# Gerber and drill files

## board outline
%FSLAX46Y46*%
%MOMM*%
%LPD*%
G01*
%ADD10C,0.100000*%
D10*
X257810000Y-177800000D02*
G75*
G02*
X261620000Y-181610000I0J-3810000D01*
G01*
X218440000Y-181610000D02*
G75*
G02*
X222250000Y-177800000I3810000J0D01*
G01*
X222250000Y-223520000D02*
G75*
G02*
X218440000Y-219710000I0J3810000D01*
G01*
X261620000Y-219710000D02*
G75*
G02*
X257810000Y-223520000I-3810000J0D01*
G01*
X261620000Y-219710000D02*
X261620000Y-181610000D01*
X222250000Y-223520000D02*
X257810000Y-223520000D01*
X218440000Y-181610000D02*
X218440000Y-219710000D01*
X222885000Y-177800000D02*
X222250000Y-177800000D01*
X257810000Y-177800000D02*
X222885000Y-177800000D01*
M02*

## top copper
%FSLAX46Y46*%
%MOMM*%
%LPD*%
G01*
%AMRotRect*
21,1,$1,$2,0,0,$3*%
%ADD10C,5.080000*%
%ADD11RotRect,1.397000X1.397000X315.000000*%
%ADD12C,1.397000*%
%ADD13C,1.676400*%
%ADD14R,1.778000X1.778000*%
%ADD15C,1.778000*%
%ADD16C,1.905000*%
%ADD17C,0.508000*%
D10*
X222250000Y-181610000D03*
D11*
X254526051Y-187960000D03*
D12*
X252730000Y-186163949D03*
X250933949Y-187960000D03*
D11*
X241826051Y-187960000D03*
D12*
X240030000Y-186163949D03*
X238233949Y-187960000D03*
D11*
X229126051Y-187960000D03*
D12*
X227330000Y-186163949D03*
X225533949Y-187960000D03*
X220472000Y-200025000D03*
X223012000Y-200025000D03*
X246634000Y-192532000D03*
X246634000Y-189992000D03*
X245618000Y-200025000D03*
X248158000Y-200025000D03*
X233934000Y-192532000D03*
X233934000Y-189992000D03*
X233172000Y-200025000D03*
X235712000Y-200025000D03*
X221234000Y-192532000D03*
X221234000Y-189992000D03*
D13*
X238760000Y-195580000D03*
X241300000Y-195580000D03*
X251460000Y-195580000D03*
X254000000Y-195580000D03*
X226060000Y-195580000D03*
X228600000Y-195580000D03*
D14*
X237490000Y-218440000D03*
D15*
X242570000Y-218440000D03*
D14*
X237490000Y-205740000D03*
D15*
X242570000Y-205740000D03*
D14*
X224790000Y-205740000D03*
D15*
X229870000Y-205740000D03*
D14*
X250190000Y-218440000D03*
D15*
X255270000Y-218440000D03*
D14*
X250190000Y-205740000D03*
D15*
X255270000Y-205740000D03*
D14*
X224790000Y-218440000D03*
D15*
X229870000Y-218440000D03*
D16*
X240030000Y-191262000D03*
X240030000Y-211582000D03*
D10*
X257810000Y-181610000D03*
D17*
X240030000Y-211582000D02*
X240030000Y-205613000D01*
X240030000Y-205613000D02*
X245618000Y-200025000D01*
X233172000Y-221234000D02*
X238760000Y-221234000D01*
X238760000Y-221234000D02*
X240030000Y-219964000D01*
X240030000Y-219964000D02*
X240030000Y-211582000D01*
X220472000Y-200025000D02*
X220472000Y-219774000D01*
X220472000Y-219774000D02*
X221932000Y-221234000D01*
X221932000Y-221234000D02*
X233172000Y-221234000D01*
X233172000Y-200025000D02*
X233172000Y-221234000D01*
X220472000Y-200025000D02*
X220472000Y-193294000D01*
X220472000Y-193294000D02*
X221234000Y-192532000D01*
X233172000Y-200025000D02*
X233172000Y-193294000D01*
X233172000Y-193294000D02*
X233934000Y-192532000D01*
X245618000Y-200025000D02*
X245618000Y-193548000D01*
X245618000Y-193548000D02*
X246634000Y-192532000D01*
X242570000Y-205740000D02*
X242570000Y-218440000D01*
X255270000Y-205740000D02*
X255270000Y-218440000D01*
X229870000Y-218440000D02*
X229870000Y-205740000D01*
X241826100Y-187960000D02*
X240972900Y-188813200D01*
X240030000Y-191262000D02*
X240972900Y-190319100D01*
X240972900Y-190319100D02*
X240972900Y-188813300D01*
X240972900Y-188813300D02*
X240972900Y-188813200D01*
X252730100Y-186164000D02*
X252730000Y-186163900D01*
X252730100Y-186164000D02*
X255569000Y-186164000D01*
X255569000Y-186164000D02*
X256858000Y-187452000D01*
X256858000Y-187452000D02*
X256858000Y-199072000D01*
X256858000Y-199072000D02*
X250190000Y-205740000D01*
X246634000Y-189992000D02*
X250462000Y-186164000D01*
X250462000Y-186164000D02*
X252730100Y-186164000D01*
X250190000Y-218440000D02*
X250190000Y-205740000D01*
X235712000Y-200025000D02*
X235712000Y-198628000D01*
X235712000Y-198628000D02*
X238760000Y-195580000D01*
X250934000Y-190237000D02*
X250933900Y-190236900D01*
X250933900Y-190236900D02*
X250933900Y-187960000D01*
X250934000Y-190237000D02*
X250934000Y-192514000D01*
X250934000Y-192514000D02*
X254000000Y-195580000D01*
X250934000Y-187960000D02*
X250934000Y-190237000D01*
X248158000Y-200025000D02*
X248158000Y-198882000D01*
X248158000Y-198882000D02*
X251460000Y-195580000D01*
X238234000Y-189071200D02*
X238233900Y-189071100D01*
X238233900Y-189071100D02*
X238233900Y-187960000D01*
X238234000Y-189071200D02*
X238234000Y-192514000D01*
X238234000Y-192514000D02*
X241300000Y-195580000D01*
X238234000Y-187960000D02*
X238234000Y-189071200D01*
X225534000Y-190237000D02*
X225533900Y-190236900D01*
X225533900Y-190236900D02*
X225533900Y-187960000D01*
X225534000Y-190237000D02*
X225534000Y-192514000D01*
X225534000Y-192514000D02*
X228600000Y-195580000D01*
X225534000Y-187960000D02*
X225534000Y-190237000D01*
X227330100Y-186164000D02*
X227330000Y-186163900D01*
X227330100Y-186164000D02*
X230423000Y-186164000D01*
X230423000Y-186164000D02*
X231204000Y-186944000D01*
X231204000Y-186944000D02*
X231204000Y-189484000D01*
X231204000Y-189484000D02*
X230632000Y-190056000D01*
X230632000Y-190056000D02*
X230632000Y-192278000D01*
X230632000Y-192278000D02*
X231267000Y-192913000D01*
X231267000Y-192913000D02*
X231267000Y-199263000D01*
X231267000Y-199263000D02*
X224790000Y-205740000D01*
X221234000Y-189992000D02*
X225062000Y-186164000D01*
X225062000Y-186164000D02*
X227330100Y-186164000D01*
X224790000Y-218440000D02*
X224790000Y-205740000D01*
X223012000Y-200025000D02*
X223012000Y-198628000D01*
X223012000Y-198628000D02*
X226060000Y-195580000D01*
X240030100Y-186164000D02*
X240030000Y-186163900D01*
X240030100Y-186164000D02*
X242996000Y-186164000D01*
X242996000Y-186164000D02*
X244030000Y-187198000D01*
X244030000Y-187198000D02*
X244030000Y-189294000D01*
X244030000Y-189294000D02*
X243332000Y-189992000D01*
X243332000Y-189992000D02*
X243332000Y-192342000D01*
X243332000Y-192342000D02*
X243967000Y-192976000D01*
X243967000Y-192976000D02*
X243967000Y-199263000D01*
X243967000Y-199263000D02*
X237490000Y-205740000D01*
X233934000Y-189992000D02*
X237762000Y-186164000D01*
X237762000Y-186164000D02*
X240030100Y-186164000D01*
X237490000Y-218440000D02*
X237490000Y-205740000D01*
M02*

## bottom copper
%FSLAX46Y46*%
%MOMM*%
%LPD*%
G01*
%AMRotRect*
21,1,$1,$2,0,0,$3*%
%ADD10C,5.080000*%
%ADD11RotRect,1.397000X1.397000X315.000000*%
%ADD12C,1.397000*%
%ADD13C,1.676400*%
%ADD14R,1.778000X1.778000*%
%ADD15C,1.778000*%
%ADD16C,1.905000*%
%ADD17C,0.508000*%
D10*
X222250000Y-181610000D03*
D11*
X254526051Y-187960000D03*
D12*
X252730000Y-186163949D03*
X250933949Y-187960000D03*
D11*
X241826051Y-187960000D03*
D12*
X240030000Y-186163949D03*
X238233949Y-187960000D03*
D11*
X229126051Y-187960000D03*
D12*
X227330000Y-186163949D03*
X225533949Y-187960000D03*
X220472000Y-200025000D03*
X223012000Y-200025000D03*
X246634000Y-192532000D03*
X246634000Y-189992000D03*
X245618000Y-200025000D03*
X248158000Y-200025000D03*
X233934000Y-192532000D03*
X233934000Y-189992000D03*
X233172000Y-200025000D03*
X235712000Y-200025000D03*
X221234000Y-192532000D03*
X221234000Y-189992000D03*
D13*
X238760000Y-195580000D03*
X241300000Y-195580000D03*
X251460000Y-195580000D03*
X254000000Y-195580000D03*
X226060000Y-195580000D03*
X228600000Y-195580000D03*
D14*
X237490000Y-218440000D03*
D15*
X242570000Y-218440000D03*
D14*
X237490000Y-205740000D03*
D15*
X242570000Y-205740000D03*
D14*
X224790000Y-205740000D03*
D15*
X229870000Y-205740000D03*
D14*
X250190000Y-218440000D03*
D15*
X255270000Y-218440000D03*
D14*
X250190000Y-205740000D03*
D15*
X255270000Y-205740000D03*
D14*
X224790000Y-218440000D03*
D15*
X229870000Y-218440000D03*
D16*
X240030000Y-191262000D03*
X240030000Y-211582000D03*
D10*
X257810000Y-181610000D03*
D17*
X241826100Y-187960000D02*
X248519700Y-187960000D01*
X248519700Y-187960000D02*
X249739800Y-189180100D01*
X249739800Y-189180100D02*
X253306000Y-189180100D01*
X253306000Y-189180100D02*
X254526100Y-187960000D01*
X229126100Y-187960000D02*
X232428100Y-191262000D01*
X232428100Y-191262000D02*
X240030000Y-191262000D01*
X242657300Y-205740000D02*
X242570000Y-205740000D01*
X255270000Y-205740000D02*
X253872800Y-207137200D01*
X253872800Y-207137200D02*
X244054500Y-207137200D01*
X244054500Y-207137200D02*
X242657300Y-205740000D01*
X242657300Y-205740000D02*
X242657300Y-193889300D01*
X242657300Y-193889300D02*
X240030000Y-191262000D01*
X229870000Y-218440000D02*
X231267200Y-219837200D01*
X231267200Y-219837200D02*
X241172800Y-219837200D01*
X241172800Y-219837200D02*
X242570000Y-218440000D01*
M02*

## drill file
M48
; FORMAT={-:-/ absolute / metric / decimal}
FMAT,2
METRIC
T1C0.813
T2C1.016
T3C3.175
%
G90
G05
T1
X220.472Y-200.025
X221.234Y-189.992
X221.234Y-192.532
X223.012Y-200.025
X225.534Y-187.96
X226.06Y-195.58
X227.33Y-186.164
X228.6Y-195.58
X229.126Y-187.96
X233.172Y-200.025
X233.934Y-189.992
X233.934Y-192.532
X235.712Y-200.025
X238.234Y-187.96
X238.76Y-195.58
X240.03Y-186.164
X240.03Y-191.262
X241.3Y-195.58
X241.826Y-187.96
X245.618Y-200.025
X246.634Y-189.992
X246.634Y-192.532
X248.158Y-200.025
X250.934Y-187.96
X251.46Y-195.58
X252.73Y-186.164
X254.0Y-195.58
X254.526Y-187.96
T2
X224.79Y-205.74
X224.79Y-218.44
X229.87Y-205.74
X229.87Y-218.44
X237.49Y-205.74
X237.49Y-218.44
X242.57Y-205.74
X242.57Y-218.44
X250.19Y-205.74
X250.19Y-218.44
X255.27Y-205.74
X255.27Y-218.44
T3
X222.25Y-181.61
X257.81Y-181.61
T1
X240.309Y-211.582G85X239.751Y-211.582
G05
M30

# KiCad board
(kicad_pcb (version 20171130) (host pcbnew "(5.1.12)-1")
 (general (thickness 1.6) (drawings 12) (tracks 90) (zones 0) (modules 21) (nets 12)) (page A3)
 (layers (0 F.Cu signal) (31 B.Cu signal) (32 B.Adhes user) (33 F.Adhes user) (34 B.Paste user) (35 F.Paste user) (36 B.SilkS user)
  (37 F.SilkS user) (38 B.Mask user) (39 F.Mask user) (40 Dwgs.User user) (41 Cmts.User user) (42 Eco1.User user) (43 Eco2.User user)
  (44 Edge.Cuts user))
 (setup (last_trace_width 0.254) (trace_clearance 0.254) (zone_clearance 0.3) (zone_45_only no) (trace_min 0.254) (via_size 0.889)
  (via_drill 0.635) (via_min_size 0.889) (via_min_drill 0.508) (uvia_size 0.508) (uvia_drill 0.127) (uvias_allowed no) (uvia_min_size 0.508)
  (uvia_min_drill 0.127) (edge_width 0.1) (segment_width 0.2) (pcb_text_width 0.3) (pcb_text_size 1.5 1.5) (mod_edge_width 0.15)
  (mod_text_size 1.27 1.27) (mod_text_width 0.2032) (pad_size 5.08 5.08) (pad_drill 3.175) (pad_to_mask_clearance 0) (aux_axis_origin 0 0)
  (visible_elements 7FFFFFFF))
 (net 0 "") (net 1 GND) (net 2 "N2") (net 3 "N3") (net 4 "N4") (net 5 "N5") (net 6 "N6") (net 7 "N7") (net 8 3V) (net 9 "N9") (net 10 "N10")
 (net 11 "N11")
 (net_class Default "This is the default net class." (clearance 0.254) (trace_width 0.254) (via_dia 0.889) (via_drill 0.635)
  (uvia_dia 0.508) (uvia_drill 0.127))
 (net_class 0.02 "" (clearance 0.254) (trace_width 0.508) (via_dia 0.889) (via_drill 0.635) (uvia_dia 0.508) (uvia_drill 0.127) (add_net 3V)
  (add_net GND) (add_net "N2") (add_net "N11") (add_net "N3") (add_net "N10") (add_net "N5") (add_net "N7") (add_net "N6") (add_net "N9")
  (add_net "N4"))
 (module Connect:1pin (layer F.Cu) (at 222.25 181.61)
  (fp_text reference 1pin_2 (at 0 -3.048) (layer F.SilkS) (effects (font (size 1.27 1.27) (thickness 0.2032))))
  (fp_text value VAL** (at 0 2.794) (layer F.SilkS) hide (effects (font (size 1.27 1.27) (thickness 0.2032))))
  (pad 1 thru_hole circle (at 0 0) (size 5.08 5.08) (drill 3.175) (layers *.Cu *.Mask F.SilkS)))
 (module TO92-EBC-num (layer F.Cu) (at 252.73 187.96 315)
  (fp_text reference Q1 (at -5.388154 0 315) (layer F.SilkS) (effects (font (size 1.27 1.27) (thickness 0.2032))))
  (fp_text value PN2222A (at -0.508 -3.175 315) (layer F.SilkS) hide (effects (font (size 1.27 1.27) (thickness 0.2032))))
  (pad 1 thru_hole rect (at 1.27 -1.27 315) (size 1.397 1.397) (drill 0.8128) (layers *.Cu *.Mask F.SilkS) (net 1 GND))
  (pad 2 thru_hole circle (at -1.27 -1.27 315) (size 1.397 1.397) (drill 0.8128) (layers *.Cu *.Mask F.SilkS) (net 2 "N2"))
  (pad 3 thru_hole circle (at -1.27 1.27 315) (size 1.397 1.397) (drill 0.8128) (layers *.Cu *.Mask F.SilkS) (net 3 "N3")))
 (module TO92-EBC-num (layer F.Cu) (at 240.03 187.96 315)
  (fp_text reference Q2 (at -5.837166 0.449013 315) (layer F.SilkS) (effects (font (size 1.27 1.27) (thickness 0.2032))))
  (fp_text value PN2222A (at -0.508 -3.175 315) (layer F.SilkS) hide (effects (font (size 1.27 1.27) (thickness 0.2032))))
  (pad 1 thru_hole rect (at 1.27 -1.27 315) (size 1.397 1.397) (drill 0.8128) (layers *.Cu *.Mask F.SilkS) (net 1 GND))
  (pad 2 thru_hole circle (at -1.27 -1.27 315) (size 1.397 1.397) (drill 0.8128) (layers *.Cu *.Mask F.SilkS) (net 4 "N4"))
  (pad 3 thru_hole circle (at -1.27 1.27 315) (size 1.397 1.397) (drill 0.8128) (layers *.Cu *.Mask F.SilkS) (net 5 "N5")))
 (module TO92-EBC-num (layer F.Cu) (at 227.33 187.96 315)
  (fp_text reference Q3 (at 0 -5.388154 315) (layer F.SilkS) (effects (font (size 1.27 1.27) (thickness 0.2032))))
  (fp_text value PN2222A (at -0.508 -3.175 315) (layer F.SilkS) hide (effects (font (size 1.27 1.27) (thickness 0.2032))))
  (pad 1 thru_hole rect (at 1.27 -1.27 315) (size 1.397 1.397) (drill 0.8128) (layers *.Cu *.Mask F.SilkS) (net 1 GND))
  (pad 2 thru_hole circle (at -1.27 -1.27 315) (size 1.397 1.397) (drill 0.8128) (layers *.Cu *.Mask F.SilkS) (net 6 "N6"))
  (pad 3 thru_hole circle (at -1.27 1.27 315) (size 1.397 1.397) (drill 0.8128) (layers *.Cu *.Mask F.SilkS) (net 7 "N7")))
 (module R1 (layer F.Cu) (at 221.742 200.025) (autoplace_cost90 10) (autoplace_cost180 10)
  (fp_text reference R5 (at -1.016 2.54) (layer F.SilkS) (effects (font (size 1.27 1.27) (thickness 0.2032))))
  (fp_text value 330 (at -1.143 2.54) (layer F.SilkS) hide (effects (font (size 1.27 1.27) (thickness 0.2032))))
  (pad 1 thru_hole circle (at -1.27 0) (size 1.397 1.397) (drill 0.8128) (layers *.Cu *.Mask F.SilkS) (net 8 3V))
  (pad 2 thru_hole circle (at 1.27 0) (size 1.397 1.397) (drill 0.8128) (layers *.Cu *.Mask F.SilkS) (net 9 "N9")))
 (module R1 (layer F.Cu) (at 246.634 191.262 90) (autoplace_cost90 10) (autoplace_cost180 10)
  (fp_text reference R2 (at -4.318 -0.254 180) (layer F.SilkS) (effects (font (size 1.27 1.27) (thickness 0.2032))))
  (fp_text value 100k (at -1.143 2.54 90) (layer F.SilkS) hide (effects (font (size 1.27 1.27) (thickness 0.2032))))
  (pad 1 thru_hole circle (at -1.27 0 90) (size 1.397 1.397) (drill 0.8128) (layers *.Cu *.Mask F.SilkS) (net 8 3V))
  (pad 2 thru_hole circle (at 1.27 0 90) (size 1.397 1.397) (drill 0.8128) (layers *.Cu *.Mask F.SilkS) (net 2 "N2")))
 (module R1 (layer F.Cu) (at 246.888 200.025) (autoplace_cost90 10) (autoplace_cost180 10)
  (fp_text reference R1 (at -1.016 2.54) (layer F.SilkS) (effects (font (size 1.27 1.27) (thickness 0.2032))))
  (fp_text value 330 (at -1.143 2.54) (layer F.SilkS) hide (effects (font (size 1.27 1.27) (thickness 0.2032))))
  (pad 1 thru_hole circle (at -1.27 0) (size 1.397 1.397) (drill 0.8128) (layers *.Cu *.Mask F.SilkS) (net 8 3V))
  (pad 2 thru_hole circle (at 1.27 0) (size 1.397 1.397) (drill 0.8128) (layers *.Cu *.Mask F.SilkS) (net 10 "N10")))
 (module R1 (layer F.Cu) (at 233.934 191.262 90) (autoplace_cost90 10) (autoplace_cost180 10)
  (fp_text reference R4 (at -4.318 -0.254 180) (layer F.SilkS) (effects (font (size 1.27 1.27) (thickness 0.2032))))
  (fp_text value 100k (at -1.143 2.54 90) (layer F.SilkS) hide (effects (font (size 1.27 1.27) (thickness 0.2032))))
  (pad 1 thru_hole circle (at -1.27 0 90) (size 1.397 1.397) (drill 0.8128) (layers *.Cu *.Mask F.SilkS) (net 8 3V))
  (pad 2 thru_hole circle (at 1.27 0 90) (size 1.397 1.397) (drill 0.8128) (layers *.Cu *.Mask F.SilkS) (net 4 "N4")))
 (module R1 (layer F.Cu) (at 234.442 200.025) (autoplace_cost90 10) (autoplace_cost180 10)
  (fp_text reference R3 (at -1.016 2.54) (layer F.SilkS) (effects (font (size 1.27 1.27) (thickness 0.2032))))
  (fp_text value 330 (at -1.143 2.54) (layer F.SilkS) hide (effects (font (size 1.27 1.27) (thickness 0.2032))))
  (pad 1 thru_hole circle (at -1.27 0) (size 1.397 1.397) (drill 0.8128) (layers *.Cu *.Mask F.SilkS) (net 8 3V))
  (pad 2 thru_hole circle (at 1.27 0) (size 1.397 1.397) (drill 0.8128) (layers *.Cu *.Mask F.SilkS) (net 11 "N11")))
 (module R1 (layer F.Cu) (at 221.234 191.262 90) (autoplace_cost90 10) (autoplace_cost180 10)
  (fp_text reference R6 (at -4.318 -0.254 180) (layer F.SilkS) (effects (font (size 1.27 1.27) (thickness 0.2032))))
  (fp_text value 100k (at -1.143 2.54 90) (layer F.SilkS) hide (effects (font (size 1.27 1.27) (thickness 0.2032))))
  (pad 1 thru_hole circle (at -1.27 0 90) (size 1.397 1.397) (drill 0.8128) (layers *.Cu *.Mask F.SilkS) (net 8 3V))
  (pad 2 thru_hole circle (at 1.27 0 90) (size 1.397 1.397) (drill 0.8128) (layers *.Cu *.Mask F.SilkS) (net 6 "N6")))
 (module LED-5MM (layer F.Cu) (at 240.03 195.58)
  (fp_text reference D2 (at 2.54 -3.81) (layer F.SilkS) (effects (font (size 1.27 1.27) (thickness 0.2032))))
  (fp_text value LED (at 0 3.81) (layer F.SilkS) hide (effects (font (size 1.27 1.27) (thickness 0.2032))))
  (pad 1 thru_hole circle (at -1.27 0) (size 1.6764 1.6764) (drill 0.8128) (layers *.Cu *.Mask F.SilkS) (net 11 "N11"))
  (pad 2 thru_hole circle (at 1.27 0) (size 1.6764 1.6764) (drill 0.8128) (layers *.Cu *.Mask F.SilkS) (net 5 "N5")))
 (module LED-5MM (layer F.Cu) (at 252.73 195.58)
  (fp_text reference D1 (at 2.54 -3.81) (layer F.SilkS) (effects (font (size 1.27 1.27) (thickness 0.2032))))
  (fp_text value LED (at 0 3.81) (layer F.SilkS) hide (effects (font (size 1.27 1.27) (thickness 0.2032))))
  (pad 1 thru_hole circle (at -1.27 0) (size 1.6764 1.6764) (drill 0.8128) (layers *.Cu *.Mask F.SilkS) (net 10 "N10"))
  (pad 2 thru_hole circle (at 1.27 0) (size 1.6764 1.6764) (drill 0.8128) (layers *.Cu *.Mask F.SilkS) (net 3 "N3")))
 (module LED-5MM (layer F.Cu) (at 227.33 195.58)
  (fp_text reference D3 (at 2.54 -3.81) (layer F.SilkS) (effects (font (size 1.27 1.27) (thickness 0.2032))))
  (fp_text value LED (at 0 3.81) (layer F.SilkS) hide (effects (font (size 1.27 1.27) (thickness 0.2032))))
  (pad 1 thru_hole circle (at -1.27 0) (size 1.6764 1.6764) (drill 0.8128) (layers *.Cu *.Mask F.SilkS) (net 9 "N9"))
  (pad 2 thru_hole circle (at 1.27 0) (size 1.6764 1.6764) (drill 0.8128) (layers *.Cu *.Mask F.SilkS) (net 7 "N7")))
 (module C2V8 (layer F.Cu) (at 240.03 218.44)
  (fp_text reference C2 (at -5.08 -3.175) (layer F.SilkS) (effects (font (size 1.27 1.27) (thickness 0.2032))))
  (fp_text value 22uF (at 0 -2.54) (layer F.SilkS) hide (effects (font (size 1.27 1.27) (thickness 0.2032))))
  (pad 1 thru_hole rect (at -2.54 0) (size 1.778 1.778) (drill 1.016) (layers *.Cu *.Mask F.SilkS) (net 4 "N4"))
  (pad 2 thru_hole circle (at 2.54 0) (size 1.778 1.778) (drill 1.016) (layers *.Cu *.Mask F.SilkS) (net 1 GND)))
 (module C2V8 (layer F.Cu) (at 240.03 205.74)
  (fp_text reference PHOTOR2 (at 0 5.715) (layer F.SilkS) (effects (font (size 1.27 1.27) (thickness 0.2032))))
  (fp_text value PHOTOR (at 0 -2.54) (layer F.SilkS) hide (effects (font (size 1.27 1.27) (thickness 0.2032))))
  (pad 1 thru_hole rect (at -2.54 0) (size 1.778 1.778) (drill 1.016) (layers *.Cu *.Mask F.SilkS) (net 4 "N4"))
  (pad 2 thru_hole circle (at 2.54 0) (size 1.778 1.778) (drill 1.016) (layers *.Cu *.Mask F.SilkS) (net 1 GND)))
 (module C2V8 (layer F.Cu) (at 227.33 205.74)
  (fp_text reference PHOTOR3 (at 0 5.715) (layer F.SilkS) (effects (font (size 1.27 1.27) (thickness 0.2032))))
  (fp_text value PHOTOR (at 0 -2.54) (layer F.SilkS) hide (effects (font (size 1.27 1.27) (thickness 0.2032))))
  (pad 1 thru_hole rect (at -2.54 0) (size 1.778 1.778) (drill 1.016) (layers *.Cu *.Mask F.SilkS) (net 6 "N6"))
  (pad 2 thru_hole circle (at 2.54 0) (size 1.778 1.778) (drill 1.016) (layers *.Cu *.Mask F.SilkS) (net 1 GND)))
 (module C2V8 (layer F.Cu) (at 252.73 218.44)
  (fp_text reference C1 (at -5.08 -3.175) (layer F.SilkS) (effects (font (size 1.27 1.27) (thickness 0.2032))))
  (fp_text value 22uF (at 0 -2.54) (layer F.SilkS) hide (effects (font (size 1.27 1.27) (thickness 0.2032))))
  (pad 1 thru_hole rect (at -2.54 0) (size 1.778 1.778) (drill 1.016) (layers *.Cu *.Mask F.SilkS) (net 2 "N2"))
  (pad 2 thru_hole circle (at 2.54 0) (size 1.778 1.778) (drill 1.016) (layers *.Cu *.Mask F.SilkS) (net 1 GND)))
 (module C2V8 (layer F.Cu) (at 252.73 205.74)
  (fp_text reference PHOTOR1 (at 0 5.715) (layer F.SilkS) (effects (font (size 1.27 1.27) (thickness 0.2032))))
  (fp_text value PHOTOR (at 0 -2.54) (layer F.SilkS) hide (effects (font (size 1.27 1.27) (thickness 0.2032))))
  (pad 1 thru_hole rect (at -2.54 0) (size 1.778 1.778) (drill 1.016) (layers *.Cu *.Mask F.SilkS) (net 2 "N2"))
  (pad 2 thru_hole circle (at 2.54 0) (size 1.778 1.778) (drill 1.016) (layers *.Cu *.Mask F.SilkS) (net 1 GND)))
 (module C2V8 (layer F.Cu) (at 227.33 218.44)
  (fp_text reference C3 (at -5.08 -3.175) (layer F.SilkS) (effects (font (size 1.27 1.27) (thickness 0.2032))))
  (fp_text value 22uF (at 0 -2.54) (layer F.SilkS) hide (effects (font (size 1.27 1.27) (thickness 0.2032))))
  (pad 1 thru_hole rect (at -2.54 0) (size 1.778 1.778) (drill 1.016) (layers *.Cu *.Mask F.SilkS) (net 6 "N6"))
  (pad 2 thru_hole circle (at 2.54 0) (size 1.778 1.778) (drill 1.016) (layers *.Cu *.Mask F.SilkS) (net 1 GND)))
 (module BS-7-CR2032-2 (layer B.Cu) (at 240.03 195.072 270)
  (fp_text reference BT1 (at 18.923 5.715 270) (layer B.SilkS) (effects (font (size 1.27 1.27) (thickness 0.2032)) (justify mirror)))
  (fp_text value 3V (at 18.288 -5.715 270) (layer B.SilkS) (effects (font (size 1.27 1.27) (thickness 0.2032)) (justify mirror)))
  (pad 2 thru_hole circle (at -3.81 0 270) (size 1.905 1.905) (drill 0.8128) (layers *.Cu *.Mask B.SilkS) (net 1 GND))
  (pad 1 thru_hole circle (at 16.51 0 270) (size 1.905 1.905) (drill oval 0.8128 1.3716) (layers *.Cu *.Mask B.SilkS) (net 8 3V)))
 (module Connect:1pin (layer F.Cu) (at 257.81 181.61)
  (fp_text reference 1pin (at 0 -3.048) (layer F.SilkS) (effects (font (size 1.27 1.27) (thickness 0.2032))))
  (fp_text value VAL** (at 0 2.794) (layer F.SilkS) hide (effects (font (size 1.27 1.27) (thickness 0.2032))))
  (pad 1 thru_hole circle (at 0 0) (size 5.08 5.08) (drill 3.175) (layers *.Cu *.Mask F.SilkS)))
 (gr_arc (start 257.81 181.61) (end 257.81 177.8) (angle 90) (layer Edge.Cuts) (width 0.1))
 (gr_arc (start 222.25 181.61) (end 218.44 181.61) (angle 90) (layer Edge.Cuts) (width 0.1))
 (gr_arc (start 222.25 219.71) (end 222.25 223.52) (angle 90) (layer Edge.Cuts) (width 0.1))
 (gr_arc (start 257.81 219.71) (end 261.62 219.71) (angle 90) (layer Edge.Cuts) (width 0.1))
 (gr_line (start 261.62 219.71) (end 261.62 181.61) (angle 90) (layer Edge.Cuts) (width 0.1))
 (gr_line (start 222.25 223.52) (end 257.81 223.52) (angle 90) (layer Edge.Cuts) (width 0.1))
 (gr_line (start 218.44 181.61) (end 218.44 219.71) (angle 90) (layer Edge.Cuts) (width 0.1))
 (gr_line (start 222.885 177.8) (end 222.25 177.8) (angle 90) (layer Edge.Cuts) (width 0.1))
 (gr_line (start 257.81 177.8) (end 222.885 177.8) (angle 90) (layer Edge.Cuts) (width 0.1))
 (segment (start 240.03 211.582) (end 240.03 205.613) (width 0.508) (layer F.Cu) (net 8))
 (segment (start 240.03 205.613) (end 245.618 200.025) (width 0.508) (layer F.Cu) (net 8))
 (segment (start 233.172 221.234) (end 238.76 221.234) (width 0.508) (layer F.Cu) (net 8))
 (segment (start 238.76 221.234) (end 240.03 219.964) (width 0.508) (layer F.Cu) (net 8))
 (segment (start 240.03 219.964) (end 240.03 211.582) (width 0.508) (layer F.Cu) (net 8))
 (segment (start 220.472 200.025) (end 220.472 219.774) (width 0.508) (layer F.Cu) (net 8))
 (segment (start 220.472 219.774) (end 221.932 221.234) (width 0.508) (layer F.Cu) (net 8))
 (segment (start 221.932 221.234) (end 233.172 221.234) (width 0.508) (layer F.Cu) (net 8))
 (segment (start 233.172 200.025) (end 233.172 221.234) (width 0.508) (layer F.Cu) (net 8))
 (segment (start 220.472 200.025) (end 220.472 193.294) (width 0.508) (layer F.Cu) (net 8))
 (segment (start 220.472 193.294) (end 221.234 192.532) (width 0.508) (layer F.Cu) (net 8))
 (segment (start 233.172 200.025) (end 233.172 193.294) (width 0.508) (layer F.Cu) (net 8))
 (segment (start 233.172 193.294) (end 233.934 192.532) (width 0.508) (layer F.Cu) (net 8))
 (segment (start 245.618 200.025) (end 245.618 193.548) (width 0.508) (layer F.Cu) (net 8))
 (segment (start 245.618 193.548) (end 246.634 192.532) (width 0.508) (layer F.Cu) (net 8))
 (segment (start 241.8261 187.96) (end 248.5197 187.96) (width 0.508) (layer B.Cu) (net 1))
 (segment (start 248.5197 187.96) (end 249.7398 189.1801) (width 0.508) (layer B.Cu) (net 1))
 (segment (start 249.7398 189.1801) (end 253.306 189.1801) (width 0.508) (layer B.Cu) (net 1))
 (segment (start 253.306 189.1801) (end 254.5261 187.96) (width 0.508) (layer B.Cu) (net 1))
 (segment (start 229.1261 187.96) (end 232.4281 191.262) (width 0.508) (layer B.Cu) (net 1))
 (segment (start 232.4281 191.262) (end 240.03 191.262) (width 0.508) (layer B.Cu) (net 1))
 (segment (start 242.6573 205.74) (end 242.57 205.74) (width 0.508) (layer B.Cu) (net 1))
 (segment (start 255.27 205.74) (end 253.8728 207.1372) (width 0.508) (layer B.Cu) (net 1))
 (segment (start 253.8728 207.1372) (end 244.0545 207.1372) (width 0.508) (layer B.Cu) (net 1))
 (segment (start 244.0545 207.1372) (end 242.6573 205.74) (width 0.508) (layer B.Cu) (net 1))
 (segment (start 242.6573 205.74) (end 242.6573 193.8893) (width 0.508) (layer B.Cu) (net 1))
 (segment (start 242.6573 193.8893) (end 240.03 191.262) (width 0.508) (layer B.Cu) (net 1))
 (segment (start 242.57 205.74) (end 242.57 218.44) (width 0.508) (layer F.Cu) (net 1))
 (segment (start 229.87 218.44) (end 231.2672 219.8372) (width 0.508) (layer B.Cu) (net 1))
 (segment (start 231.2672 219.8372) (end 241.1728 219.8372) (width 0.508) (layer B.Cu) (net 1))
 (segment (start 241.1728 219.8372) (end 242.57 218.44) (width 0.508) (layer B.Cu) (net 1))
 (segment (start 255.27 205.74) (end 255.27 218.44) (width 0.508) (layer F.Cu) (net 1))
 (segment (start 229.87 218.44) (end 229.87 205.74) (width 0.508) (layer F.Cu) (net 1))
 (segment (start 241.8261 187.96) (end 240.9729 188.8132) (width 0.508) (layer F.Cu) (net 1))
 (segment (start 240.03 191.262) (end 240.9729 190.3191) (width 0.508) (layer F.Cu) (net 1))
 (segment (start 240.9729 190.3191) (end 240.9729 188.8133) (width 0.508) (layer F.Cu) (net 1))
 (segment (start 240.9729 188.8133) (end 240.9729 188.8132) (width 0.508) (layer F.Cu) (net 1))
 (segment (start 252.7301 186.164) (end 252.73 186.1639) (width 0.508) (layer F.Cu) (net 2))
 (segment (start 252.7301 186.164) (end 255.569 186.164) (width 0.508) (layer F.Cu) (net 2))
 (segment (start 255.569 186.164) (end 256.858 187.452) (width 0.508) (layer F.Cu) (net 2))
 (segment (start 256.858 187.452) (end 256.858 199.072) (width 0.508) (layer F.Cu) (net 2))
 (segment (start 256.858 199.072) (end 250.19 205.74) (width 0.508) (layer F.Cu) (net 2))
 (segment (start 246.634 189.992) (end 250.462 186.164) (width 0.508) (layer F.Cu) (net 2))
 (segment (start 250.462 186.164) (end 252.7301 186.164) (width 0.508) (layer F.Cu) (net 2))
 (segment (start 250.19 218.44) (end 250.19 205.74) (width 0.508) (layer F.Cu) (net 2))
 (segment (start 235.712 200.025) (end 235.712 198.628) (width 0.508) (layer F.Cu) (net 11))
 (segment (start 235.712 198.628) (end 238.76 195.58) (width 0.508) (layer F.Cu) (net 11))
 (segment (start 250.934 190.237) (end 250.9339 190.2369) (width 0.508) (layer F.Cu) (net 3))
 (segment (start 250.9339 190.2369) (end 250.9339 187.96) (width 0.508) (layer F.Cu) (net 3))
 (segment (start 250.934 190.237) (end 250.934 192.514) (width 0.508) (layer F.Cu) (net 3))
 (segment (start 250.934 192.514) (end 254 195.58) (width 0.508) (layer F.Cu) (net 3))
 (segment (start 250.934 187.96) (end 250.934 190.237) (width 0.508) (layer F.Cu) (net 3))
 (segment (start 248.158 200.025) (end 248.158 198.882) (width 0.508) (layer F.Cu) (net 10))
 (segment (start 248.158 198.882) (end 251.46 195.58) (width 0.508) (layer F.Cu) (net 10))
 (segment (start 238.234 189.0712) (end 238.2339 189.0711) (width 0.508) (layer F.Cu) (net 5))
 (segment (start 238.2339 189.0711) (end 238.2339 187.96) (width 0.508) (layer F.Cu) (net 5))
 (segment (start 238.234 189.0712) (end 238.234 192.514) (width 0.508) (layer F.Cu) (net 5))
 (segment (start 238.234 192.514) (end 241.3 195.58) (width 0.508) (layer F.Cu) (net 5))
 (segment (start 238.234 187.96) (end 238.234 189.0712) (width 0.508) (layer F.Cu) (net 5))
 (segment (start 225.534 190.237) (end 225.5339 190.2369) (width 0.508) (layer F.Cu) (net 7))
 (segment (start 225.5339 190.2369) (end 225.5339 187.96) (width 0.508) (layer F.Cu) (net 7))
 (segment (start 225.534 190.237) (end 225.534 192.514) (width 0.508) (layer F.Cu) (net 7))
 (segment (start 225.534 192.514) (end 228.6 195.58) (width 0.508) (layer F.Cu) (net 7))
 (segment (start 225.534 187.96) (end 225.534 190.237) (width 0.508) (layer F.Cu) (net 7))
 (segment (start 227.3301 186.164) (end 227.33 186.1639) (width 0.508) (layer F.Cu) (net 6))
 (segment (start 227.3301 186.164) (end 230.423 186.164) (width 0.508) (layer F.Cu) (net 6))
 (segment (start 230.423 186.164) (end 231.204 186.944) (width 0.508) (layer F.Cu) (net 6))
 (segment (start 231.204 186.944) (end 231.204 189.484) (width 0.508) (layer F.Cu) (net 6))
 (segment (start 231.204 189.484) (end 230.632 190.056) (width 0.508) (layer F.Cu) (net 6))
 (segment (start 230.632 190.056) (end 230.632 192.278) (width 0.508) (layer F.Cu) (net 6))
 (segment (start 230.632 192.278) (end 231.267 192.913) (width 0.508) (layer F.Cu) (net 6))
 (segment (start 231.267 192.913) (end 231.267 199.263) (width 0.508) (layer F.Cu) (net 6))
 (segment (start 231.267 199.263) (end 224.79 205.74) (width 0.508) (layer F.Cu) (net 6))
 (segment (start 221.234 189.992) (end 225.062 186.164) (width 0.508) (layer F.Cu) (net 6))
 (segment (start 225.062 186.164) (end 227.3301 186.164) (width 0.508) (layer F.Cu) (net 6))
 (segment (start 224.79 218.44) (end 224.79 205.74) (width 0.508) (layer F.Cu) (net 6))
 (segment (start 223.012 200.025) (end 223.012 198.628) (width 0.508) (layer F.Cu) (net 9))
 (segment (start 223.012 198.628) (end 226.06 195.58) (width 0.508) (layer F.Cu) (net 9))
 (segment (start 240.0301 186.164) (end 240.03 186.1639) (width 0.508) (layer F.Cu) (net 4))
 (segment (start 240.0301 186.164) (end 242.996 186.164) (width 0.508) (layer F.Cu) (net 4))
 (segment (start 242.996 186.164) (end 244.03 187.198) (width 0.508) (layer F.Cu) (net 4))
 (segment (start 244.03 187.198) (end 244.03 189.294) (width 0.508) (layer F.Cu) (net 4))
 (segment (start 244.03 189.294) (end 243.332 189.992) (width 0.508) (layer F.Cu) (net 4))
 (segment (start 243.332 189.992) (end 243.332 192.342) (width 0.508) (layer F.Cu) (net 4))
 (segment (start 243.332 192.342) (end 243.967 192.976) (width 0.508) (layer F.Cu) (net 4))
 (segment (start 243.967 192.976) (end 243.967 199.263) (width 0.508) (layer F.Cu) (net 4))
 (segment (start 243.967 199.263) (end 237.49 205.74) (width 0.508) (layer F.Cu) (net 4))
 (segment (start 233.934 189.992) (end 237.762 186.164) (width 0.508) (layer F.Cu) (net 4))
 (segment (start 237.762 186.164) (end 240.0301 186.164) (width 0.508) (layer F.Cu) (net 4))
 (segment (start 237.49 218.44) (end 237.49 205.74) (width 0.508) (layer F.Cu) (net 4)))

